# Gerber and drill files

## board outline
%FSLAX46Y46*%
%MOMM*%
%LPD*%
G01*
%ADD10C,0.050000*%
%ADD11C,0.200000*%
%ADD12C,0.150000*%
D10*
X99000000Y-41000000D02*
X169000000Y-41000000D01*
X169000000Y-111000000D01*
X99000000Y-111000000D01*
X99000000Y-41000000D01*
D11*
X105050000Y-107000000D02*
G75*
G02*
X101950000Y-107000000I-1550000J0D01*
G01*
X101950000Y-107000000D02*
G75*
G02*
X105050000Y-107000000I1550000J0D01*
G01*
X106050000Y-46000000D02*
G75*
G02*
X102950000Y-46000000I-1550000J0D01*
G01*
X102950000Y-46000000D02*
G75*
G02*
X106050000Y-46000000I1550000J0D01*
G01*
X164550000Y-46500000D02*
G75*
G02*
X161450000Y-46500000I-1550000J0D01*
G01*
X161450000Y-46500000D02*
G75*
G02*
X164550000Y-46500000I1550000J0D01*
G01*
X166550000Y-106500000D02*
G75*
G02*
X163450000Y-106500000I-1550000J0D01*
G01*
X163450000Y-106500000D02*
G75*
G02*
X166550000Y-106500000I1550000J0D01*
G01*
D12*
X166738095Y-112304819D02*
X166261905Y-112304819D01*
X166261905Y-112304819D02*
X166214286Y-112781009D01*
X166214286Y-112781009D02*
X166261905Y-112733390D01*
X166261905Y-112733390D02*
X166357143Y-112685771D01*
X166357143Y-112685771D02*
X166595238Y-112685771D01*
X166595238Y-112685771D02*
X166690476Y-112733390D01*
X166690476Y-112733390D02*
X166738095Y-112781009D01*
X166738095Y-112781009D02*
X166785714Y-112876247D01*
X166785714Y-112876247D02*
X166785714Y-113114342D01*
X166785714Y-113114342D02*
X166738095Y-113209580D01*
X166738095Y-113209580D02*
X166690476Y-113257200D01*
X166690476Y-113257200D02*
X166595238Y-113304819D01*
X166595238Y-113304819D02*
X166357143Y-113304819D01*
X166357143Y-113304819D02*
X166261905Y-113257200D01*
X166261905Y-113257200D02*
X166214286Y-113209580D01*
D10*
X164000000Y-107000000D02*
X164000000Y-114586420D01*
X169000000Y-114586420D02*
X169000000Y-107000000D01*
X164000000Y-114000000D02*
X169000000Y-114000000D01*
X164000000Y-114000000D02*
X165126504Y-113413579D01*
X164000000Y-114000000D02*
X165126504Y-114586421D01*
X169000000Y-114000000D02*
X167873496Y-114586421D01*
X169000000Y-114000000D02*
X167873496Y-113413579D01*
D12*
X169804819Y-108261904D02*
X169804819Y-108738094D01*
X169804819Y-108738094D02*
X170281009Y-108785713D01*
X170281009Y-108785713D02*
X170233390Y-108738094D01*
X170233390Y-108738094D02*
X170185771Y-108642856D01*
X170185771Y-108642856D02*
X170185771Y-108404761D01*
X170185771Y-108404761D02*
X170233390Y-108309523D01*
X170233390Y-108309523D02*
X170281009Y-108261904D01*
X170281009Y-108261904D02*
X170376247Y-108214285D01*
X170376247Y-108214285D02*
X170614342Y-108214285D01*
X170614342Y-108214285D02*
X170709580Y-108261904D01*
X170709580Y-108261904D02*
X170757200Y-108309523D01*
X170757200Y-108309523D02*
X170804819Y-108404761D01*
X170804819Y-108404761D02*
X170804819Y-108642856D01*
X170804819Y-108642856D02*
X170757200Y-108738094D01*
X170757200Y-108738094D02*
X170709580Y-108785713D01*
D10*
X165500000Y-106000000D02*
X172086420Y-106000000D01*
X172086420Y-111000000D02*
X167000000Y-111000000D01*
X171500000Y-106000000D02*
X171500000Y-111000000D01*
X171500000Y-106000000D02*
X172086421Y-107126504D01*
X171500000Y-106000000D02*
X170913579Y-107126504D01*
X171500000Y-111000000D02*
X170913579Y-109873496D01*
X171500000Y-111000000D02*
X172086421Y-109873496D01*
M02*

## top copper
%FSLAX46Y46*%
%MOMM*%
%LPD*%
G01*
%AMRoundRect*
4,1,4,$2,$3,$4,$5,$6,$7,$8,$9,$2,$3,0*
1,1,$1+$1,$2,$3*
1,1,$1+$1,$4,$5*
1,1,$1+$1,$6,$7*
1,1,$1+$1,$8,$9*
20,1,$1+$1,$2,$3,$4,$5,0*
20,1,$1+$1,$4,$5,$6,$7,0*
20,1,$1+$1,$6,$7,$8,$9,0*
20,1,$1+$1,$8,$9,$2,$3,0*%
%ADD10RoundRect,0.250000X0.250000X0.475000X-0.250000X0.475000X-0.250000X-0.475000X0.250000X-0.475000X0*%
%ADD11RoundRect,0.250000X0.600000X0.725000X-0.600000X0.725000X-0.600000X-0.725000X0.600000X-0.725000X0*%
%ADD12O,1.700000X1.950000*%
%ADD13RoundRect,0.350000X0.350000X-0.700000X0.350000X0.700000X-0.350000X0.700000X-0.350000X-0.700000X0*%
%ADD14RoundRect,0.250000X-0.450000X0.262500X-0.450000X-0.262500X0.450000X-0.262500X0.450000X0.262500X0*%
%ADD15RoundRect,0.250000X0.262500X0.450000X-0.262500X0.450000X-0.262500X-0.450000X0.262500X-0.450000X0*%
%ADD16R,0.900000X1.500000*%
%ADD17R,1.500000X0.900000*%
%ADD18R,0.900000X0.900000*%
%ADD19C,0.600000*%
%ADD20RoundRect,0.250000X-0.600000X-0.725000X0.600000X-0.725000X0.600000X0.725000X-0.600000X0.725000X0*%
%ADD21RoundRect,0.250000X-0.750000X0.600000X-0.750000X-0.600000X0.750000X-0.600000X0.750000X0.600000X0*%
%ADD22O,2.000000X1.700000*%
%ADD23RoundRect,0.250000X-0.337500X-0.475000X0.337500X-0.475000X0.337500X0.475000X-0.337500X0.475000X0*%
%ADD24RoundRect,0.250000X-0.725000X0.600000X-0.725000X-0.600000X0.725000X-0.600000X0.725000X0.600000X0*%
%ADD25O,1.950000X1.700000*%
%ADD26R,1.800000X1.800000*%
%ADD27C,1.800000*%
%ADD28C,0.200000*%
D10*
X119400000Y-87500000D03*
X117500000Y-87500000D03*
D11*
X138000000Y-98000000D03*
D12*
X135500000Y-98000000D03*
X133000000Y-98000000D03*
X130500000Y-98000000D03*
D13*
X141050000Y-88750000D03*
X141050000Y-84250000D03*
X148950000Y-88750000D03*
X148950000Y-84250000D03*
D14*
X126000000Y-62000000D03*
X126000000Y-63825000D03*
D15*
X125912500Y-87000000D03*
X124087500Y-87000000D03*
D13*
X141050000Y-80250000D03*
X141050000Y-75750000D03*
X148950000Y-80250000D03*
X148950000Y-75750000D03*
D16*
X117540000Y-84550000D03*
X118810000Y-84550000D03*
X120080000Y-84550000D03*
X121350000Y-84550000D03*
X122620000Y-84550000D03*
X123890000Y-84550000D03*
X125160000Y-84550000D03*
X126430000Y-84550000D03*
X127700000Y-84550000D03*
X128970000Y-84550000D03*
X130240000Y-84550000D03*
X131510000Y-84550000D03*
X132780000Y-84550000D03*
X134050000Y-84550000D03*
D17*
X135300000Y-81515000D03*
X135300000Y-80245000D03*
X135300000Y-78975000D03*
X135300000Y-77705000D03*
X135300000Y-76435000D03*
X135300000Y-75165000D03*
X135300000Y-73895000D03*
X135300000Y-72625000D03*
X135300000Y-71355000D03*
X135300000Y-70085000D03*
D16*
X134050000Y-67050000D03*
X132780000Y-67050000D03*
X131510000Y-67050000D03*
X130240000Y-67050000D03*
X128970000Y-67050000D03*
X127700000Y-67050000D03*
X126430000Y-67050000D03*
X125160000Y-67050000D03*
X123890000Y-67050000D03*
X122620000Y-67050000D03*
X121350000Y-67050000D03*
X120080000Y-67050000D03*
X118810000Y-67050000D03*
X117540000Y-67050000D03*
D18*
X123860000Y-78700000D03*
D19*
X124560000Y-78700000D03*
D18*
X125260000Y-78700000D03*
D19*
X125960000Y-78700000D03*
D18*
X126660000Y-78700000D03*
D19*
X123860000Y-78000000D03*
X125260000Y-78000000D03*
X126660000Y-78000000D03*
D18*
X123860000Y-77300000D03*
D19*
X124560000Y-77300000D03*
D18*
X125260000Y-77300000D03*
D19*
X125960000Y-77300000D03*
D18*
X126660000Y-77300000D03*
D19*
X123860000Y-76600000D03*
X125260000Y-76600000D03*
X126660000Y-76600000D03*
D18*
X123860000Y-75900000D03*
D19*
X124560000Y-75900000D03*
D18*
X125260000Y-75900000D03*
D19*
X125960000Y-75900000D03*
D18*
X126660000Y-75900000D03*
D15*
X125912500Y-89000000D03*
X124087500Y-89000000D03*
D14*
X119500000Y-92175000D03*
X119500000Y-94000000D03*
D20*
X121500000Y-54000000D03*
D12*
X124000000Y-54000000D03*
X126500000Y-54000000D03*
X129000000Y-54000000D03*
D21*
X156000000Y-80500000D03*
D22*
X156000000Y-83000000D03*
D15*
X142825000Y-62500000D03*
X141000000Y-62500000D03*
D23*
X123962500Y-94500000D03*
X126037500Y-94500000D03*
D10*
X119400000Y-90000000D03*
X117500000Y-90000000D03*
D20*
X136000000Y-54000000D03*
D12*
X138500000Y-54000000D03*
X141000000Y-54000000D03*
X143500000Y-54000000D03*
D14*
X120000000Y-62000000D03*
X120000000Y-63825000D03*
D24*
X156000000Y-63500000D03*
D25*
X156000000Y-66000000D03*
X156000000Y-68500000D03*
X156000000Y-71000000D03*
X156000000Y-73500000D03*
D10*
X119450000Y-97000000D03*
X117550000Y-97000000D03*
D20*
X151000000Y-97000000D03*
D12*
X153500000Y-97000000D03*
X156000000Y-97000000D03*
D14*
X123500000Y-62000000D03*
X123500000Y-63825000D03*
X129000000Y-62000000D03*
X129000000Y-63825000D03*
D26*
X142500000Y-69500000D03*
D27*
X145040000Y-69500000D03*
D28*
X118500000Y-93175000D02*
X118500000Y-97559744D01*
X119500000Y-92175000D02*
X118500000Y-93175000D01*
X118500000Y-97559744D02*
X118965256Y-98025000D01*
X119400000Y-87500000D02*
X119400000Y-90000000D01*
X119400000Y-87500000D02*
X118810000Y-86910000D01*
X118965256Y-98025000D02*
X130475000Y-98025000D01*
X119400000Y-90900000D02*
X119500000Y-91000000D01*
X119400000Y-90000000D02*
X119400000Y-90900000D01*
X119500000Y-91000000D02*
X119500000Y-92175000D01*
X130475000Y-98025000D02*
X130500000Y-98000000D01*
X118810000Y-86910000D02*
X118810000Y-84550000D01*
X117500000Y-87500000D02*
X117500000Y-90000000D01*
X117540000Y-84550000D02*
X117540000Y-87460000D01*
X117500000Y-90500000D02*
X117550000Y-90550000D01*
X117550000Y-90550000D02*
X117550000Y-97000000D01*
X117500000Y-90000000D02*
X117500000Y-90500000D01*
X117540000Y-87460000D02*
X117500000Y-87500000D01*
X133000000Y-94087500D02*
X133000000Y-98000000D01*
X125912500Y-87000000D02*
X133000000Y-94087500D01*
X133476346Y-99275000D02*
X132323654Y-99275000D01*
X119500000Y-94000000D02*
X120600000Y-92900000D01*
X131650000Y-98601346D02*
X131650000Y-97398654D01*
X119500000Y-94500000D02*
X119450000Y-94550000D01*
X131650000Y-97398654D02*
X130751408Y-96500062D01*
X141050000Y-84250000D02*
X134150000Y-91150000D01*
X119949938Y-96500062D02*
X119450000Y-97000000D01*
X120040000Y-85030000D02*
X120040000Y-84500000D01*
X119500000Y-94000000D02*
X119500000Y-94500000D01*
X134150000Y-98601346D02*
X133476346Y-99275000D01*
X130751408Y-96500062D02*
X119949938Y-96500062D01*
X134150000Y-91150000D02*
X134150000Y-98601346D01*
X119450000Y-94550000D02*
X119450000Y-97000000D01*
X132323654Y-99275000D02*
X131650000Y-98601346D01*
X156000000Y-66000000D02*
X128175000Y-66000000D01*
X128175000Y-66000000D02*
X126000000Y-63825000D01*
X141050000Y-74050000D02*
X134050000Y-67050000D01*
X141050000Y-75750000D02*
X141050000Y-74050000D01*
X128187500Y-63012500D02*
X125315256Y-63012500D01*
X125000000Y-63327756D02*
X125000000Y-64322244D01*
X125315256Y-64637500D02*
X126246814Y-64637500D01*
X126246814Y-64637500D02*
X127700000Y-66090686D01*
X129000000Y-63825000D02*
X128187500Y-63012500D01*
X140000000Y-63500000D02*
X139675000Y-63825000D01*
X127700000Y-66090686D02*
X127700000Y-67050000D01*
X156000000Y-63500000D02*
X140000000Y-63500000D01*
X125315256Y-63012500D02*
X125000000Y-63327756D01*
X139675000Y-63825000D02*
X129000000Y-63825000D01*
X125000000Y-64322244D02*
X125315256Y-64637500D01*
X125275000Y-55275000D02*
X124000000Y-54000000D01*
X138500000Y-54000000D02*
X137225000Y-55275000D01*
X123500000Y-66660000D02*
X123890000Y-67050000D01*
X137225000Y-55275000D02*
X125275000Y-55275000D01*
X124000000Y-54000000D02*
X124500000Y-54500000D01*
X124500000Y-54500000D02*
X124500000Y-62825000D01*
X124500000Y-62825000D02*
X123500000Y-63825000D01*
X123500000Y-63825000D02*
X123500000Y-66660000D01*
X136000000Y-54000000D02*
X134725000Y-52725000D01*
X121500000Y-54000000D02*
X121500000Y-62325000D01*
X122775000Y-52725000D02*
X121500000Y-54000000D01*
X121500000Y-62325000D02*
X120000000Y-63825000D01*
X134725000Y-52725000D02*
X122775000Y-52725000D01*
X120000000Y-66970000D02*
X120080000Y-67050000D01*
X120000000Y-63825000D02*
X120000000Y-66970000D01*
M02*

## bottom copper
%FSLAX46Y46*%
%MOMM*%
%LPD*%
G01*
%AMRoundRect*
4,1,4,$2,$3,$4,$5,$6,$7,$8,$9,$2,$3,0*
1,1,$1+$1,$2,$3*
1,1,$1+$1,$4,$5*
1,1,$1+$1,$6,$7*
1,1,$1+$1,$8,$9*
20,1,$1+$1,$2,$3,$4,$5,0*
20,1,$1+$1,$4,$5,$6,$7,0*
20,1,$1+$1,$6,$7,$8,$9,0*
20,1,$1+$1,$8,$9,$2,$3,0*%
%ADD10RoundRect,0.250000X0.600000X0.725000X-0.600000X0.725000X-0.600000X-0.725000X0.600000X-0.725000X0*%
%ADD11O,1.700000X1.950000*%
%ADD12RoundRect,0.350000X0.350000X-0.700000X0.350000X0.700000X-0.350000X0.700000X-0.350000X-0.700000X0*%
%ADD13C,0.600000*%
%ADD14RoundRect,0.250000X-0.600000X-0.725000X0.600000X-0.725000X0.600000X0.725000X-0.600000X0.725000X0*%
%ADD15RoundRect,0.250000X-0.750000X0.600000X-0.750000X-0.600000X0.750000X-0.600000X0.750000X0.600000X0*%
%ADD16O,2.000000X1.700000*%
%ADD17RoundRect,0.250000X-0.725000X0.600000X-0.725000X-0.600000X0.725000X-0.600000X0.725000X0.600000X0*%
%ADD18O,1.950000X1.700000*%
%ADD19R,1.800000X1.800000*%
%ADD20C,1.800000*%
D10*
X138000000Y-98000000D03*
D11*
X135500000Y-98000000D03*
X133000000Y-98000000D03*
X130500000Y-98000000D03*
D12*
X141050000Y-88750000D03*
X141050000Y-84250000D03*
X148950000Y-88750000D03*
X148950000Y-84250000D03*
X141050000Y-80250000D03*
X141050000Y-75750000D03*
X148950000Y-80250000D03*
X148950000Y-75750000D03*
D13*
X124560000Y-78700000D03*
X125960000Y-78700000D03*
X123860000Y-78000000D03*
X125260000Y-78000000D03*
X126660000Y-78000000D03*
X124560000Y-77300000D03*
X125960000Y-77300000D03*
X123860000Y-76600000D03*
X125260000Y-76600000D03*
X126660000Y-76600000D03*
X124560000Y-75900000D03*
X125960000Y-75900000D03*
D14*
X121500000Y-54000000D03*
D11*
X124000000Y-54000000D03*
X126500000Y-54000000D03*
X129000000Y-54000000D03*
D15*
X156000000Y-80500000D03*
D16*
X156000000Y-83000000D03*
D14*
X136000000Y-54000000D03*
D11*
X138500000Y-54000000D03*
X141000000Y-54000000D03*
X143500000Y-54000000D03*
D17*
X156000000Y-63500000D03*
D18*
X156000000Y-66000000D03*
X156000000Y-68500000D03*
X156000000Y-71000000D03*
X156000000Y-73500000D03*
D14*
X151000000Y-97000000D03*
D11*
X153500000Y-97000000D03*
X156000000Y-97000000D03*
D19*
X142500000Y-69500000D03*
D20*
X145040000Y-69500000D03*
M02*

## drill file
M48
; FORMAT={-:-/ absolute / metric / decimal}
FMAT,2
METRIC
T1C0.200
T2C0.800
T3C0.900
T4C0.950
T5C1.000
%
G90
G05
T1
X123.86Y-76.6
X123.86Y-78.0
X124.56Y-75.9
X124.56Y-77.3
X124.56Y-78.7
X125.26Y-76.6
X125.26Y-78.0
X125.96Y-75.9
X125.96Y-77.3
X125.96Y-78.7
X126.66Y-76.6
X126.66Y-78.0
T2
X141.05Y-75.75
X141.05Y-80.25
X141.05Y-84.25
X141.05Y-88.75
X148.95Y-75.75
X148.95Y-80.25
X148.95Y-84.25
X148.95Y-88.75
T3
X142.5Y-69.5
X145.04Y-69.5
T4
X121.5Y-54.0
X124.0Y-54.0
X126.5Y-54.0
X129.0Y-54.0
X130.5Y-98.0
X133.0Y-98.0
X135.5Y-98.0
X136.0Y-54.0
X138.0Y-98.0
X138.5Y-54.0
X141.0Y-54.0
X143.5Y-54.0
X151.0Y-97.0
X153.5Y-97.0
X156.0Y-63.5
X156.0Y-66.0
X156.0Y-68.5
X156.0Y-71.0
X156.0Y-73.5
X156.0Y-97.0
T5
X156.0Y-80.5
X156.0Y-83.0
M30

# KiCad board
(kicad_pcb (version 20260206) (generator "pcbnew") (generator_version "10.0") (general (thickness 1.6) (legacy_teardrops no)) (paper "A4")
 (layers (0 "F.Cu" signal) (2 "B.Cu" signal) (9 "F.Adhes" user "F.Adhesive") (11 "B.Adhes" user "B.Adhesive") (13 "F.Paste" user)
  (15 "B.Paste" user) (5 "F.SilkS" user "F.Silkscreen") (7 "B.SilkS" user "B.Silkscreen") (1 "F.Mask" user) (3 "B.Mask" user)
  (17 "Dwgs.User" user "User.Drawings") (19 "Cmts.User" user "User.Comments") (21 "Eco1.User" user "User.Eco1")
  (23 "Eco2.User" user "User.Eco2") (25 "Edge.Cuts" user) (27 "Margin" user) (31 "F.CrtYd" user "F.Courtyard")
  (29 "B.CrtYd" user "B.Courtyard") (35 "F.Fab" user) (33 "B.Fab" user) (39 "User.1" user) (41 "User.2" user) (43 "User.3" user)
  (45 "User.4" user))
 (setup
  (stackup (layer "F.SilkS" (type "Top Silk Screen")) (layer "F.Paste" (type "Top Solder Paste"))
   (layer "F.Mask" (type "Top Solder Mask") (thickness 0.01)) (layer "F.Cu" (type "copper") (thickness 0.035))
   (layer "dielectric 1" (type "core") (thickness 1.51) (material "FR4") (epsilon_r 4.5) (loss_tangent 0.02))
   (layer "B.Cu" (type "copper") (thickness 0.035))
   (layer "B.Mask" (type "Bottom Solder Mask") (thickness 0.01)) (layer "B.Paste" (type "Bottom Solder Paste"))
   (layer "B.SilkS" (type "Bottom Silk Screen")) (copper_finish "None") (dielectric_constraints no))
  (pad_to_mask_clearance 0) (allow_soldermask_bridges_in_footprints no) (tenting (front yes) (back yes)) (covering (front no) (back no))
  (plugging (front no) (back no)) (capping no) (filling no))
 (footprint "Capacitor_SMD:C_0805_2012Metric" (layer "F.Cu") (at 118.45 87.5 180)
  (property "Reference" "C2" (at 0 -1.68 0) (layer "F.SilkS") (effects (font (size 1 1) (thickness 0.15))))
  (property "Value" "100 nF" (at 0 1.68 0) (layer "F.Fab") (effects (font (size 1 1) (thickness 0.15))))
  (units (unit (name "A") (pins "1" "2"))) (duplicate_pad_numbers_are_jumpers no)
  (pad "1" smd roundrect (at -0.95 0 180) (size 1 1.45) (layers "F.Cu" "F.Mask" "F.Paste") (roundrect_rratio 0.25) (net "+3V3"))
  (pad "2" smd roundrect (at 0.95 0 180) (size 1 1.45) (layers "F.Cu" "F.Mask" "F.Paste") (roundrect_rratio 0.25) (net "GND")))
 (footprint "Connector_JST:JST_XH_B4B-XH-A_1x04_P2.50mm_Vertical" (layer "F.Cu") (at 138 98 180)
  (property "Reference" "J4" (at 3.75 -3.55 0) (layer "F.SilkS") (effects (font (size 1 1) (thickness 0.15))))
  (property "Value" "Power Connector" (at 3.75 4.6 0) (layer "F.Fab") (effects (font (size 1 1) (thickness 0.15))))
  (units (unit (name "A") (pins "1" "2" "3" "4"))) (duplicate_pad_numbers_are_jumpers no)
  (pad "1" thru_hole roundrect (at 0 0 180) (size 1.7 1.95) (drill 0.95) (layers "*.Cu" "*.Mask") (remove_unused_layers no)
   (roundrect_rratio 0.147059) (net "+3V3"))
  (pad "2" thru_hole oval (at 2.5 0 180) (size 1.7 1.95) (drill 0.95) (layers "*.Cu" "*.Mask") (remove_unused_layers no) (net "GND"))
  (pad "3" thru_hole oval (at 5 0 180) (size 1.7 1.95) (drill 0.95) (layers "*.Cu" "*.Mask") (remove_unused_layers no) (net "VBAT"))
  (pad "4" thru_hole oval (at 7.5 0 180) (size 1.7 1.95) (drill 0.95) (layers "*.Cu" "*.Mask") (remove_unused_layers no) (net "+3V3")))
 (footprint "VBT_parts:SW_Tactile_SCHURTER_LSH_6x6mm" (layer "F.Cu") (at 145 86.5)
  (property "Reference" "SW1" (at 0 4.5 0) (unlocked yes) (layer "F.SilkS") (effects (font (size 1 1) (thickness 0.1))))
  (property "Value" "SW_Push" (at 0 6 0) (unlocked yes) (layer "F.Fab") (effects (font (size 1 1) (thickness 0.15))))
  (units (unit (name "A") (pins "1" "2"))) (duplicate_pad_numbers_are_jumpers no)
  (pad "1" thru_hole roundrect (at -3.95 2.25 90) (size 2.1 1.4) (drill 0.8) (layers "*.Cu" "*.Mask") (remove_unused_layers no)
   (roundrect_rratio 0.25) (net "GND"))
  (pad "2" thru_hole roundrect (at -3.95 -2.25 90) (size 2.1 1.4) (drill 0.8) (layers "*.Cu" "*.Mask") (remove_unused_layers no)
   (roundrect_rratio 0.25) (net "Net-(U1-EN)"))
  (pad "3" thru_hole roundrect (at 3.95 2.25 90) (size 2.1 1.4) (drill 0.8) (layers "*.Cu" "*.Mask") (remove_unused_layers no)
   (roundrect_rratio 0.25))
  (pad "4" thru_hole roundrect (at 3.95 -2.25 90) (size 2.1 1.4) (drill 0.8) (layers "*.Cu" "*.Mask") (remove_unused_layers no)
   (roundrect_rratio 0.25)))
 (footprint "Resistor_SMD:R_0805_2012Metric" (layer "F.Cu") (at 126 62.9125 -90)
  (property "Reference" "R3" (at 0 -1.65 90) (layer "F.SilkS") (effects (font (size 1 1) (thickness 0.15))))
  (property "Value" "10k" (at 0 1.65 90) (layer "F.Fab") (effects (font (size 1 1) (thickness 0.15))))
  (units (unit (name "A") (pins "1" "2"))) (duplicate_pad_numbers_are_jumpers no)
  (pad "1" smd roundrect (at -0.9125 0 270) (size 1.025 1.4) (layers "F.Cu" "F.Mask" "F.Paste") (roundrect_rratio 0.243902) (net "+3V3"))
  (pad "2" smd roundrect (at 0.9125 0 270) (size 1.025 1.4) (layers "F.Cu" "F.Mask" "F.Paste") (roundrect_rratio 0.243902) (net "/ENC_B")))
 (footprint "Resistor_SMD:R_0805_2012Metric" (layer "F.Cu") (at 125 87 180)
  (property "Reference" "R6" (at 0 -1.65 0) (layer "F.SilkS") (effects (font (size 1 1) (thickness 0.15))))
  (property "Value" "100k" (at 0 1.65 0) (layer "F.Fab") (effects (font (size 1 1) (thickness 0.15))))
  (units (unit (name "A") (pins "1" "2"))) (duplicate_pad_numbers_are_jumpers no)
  (pad "1" smd roundrect (at -0.9125 0 180) (size 1.025 1.4) (layers "F.Cu" "F.Mask" "F.Paste") (roundrect_rratio 0.243902) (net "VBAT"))
  (pad "2" smd roundrect (at 0.9125 0 180) (size 1.025 1.4) (layers "F.Cu" "F.Mask" "F.Paste") (roundrect_rratio 0.243902)
   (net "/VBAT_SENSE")))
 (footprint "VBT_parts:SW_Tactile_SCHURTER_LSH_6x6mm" (layer "F.Cu") (at 145 78)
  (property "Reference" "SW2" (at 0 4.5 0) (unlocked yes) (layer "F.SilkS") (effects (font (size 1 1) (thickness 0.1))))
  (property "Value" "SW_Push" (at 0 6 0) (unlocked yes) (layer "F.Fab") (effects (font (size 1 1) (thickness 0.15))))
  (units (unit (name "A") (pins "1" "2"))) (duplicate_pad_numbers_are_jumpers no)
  (pad "1" thru_hole roundrect (at -3.95 2.25 90) (size 2.1 1.4) (drill 0.8) (layers "*.Cu" "*.Mask") (remove_unused_layers no)
   (roundrect_rratio 0.25) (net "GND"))
  (pad "2" thru_hole roundrect (at -3.95 -2.25 90) (size 2.1 1.4) (drill 0.8) (layers "*.Cu" "*.Mask") (remove_unused_layers no)
   (roundrect_rratio 0.25) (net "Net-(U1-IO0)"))
  (pad "3" thru_hole roundrect (at 3.95 2.25 90) (size 2.1 1.4) (drill 0.8) (layers "*.Cu" "*.Mask") (remove_unused_layers no)
   (roundrect_rratio 0.25))
  (pad "4" thru_hole roundrect (at 3.95 -2.25 90) (size 2.1 1.4) (drill 0.8) (layers "*.Cu" "*.Mask") (remove_unused_layers no)
   (roundrect_rratio 0.25)))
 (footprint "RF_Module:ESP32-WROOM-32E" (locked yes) (layer "F.Cu") (at 122.8 75.8 90)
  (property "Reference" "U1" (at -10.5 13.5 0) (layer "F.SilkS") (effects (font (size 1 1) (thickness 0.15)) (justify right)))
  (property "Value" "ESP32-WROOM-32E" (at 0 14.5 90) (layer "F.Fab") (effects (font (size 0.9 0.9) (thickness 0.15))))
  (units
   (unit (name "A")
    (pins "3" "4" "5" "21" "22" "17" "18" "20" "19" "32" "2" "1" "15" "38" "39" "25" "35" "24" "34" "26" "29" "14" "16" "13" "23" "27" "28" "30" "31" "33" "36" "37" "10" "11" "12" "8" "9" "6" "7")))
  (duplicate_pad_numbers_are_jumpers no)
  (pad "1" smd rect (at -8.75 -5.26 90) (size 1.5 0.9) (layers "F.Cu" "F.Mask" "F.Paste") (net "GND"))
  (pad "2" smd rect (at -8.75 -3.99 90) (size 1.5 0.9) (layers "F.Cu" "F.Mask" "F.Paste") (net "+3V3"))
  (pad "3" smd rect (at -8.75 -2.72 90) (size 1.5 0.9) (layers "F.Cu" "F.Mask" "F.Paste") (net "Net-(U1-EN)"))
  (pad "4" smd rect (at -8.75 -1.45 90) (size 1.5 0.9) (layers "F.Cu" "F.Mask" "F.Paste") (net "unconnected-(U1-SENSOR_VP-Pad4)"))
  (pad "5" smd rect (at -8.75 -0.18 90) (size 1.5 0.9) (layers "F.Cu" "F.Mask" "F.Paste") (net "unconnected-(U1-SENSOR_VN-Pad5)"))
  (pad "6" smd rect (at -8.75 1.09 90) (size 1.5 0.9) (layers "F.Cu" "F.Mask" "F.Paste") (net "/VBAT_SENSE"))
  (pad "7" smd rect (at -8.75 2.36 90) (size 1.5 0.9) (layers "F.Cu" "F.Mask" "F.Paste") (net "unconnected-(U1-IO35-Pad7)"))
  (pad "8" smd rect (at -8.75 3.63 90) (size 1.5 0.9) (layers "F.Cu" "F.Mask" "F.Paste") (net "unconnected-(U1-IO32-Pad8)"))
  (pad "9" smd rect (at -8.75 4.9 90) (size 1.5 0.9) (layers "F.Cu" "F.Mask" "F.Paste") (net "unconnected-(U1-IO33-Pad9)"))
  (pad "10" smd rect (at -8.75 6.17 90) (size 1.5 0.9) (layers "F.Cu" "F.Mask" "F.Paste") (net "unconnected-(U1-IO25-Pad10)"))
  (pad "11" smd rect (at -8.75 7.44 90) (size 1.5 0.9) (layers "F.Cu" "F.Mask" "F.Paste") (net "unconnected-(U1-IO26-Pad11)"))
  (pad "12" smd rect (at -8.75 8.71 90) (size 1.5 0.9) (layers "F.Cu" "F.Mask" "F.Paste") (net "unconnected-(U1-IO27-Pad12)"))
  (pad "13" smd rect (at -8.75 9.98 90) (size 1.5 0.9) (layers "F.Cu" "F.Mask" "F.Paste") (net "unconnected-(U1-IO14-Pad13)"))
  (pad "14" smd rect (at -8.75 11.25 90) (size 1.5 0.9) (layers "F.Cu" "F.Mask" "F.Paste") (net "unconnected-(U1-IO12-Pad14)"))
  (pad "15" smd rect (at -5.715 12.5 180) (size 1.5 0.9) (layers "F.Cu" "F.Mask" "F.Paste") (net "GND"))
  (pad "16" smd rect (at -4.445 12.5 180) (size 1.5 0.9) (layers "F.Cu" "F.Mask" "F.Paste") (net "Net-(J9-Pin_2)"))
  (pad "17" smd rect (at -3.175 12.5 180) (size 1.5 0.9) (layers "F.Cu" "F.Mask" "F.Paste") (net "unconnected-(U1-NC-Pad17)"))
  (pad "18" smd rect (at -1.905 12.5 180) (size 1.5 0.9) (layers "F.Cu" "F.Mask" "F.Paste") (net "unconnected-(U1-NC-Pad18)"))
  (pad "19" smd rect (at -0.635 12.5 180) (size 1.5 0.9) (layers "F.Cu" "F.Mask" "F.Paste") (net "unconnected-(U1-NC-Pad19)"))
  (pad "20" smd rect (at 0.635 12.5 180) (size 1.5 0.9) (layers "F.Cu" "F.Mask" "F.Paste") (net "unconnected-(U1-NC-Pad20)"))
  (pad "21" smd rect (at 1.905 12.5 180) (size 1.5 0.9) (layers "F.Cu" "F.Mask" "F.Paste") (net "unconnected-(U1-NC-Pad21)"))
  (pad "22" smd rect (at 3.175 12.5 180) (size 1.5 0.9) (layers "F.Cu" "F.Mask" "F.Paste") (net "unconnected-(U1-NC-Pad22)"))
  (pad "23" smd rect (at 4.445 12.5 180) (size 1.5 0.9) (layers "F.Cu" "F.Mask" "F.Paste") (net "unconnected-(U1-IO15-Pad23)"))
  (pad "24" smd rect (at 5.715 12.5 180) (size 1.5 0.9) (layers "F.Cu" "F.Mask" "F.Paste") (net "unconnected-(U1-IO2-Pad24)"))
  (pad "25" smd rect (at 8.75 11.25 90) (size 1.5 0.9) (layers "F.Cu" "F.Mask" "F.Paste") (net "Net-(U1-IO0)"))
  (pad "26" smd rect (at 8.75 9.98 90) (size 1.5 0.9) (layers "F.Cu" "F.Mask" "F.Paste") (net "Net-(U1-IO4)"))
  (pad "27" smd rect (at 8.75 8.71 90) (size 1.5 0.9) (layers "F.Cu" "F.Mask" "F.Paste") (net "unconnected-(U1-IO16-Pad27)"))
  (pad "28" smd rect (at 8.75 7.44 90) (size 1.5 0.9) (layers "F.Cu" "F.Mask" "F.Paste") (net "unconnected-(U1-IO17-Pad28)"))
  (pad "29" smd rect (at 8.75 6.17 90) (size 1.5 0.9) (layers "F.Cu" "F.Mask" "F.Paste") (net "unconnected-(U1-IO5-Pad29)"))
  (pad "30" smd rect (at 8.75 4.9 90) (size 1.5 0.9) (layers "F.Cu" "F.Mask" "F.Paste") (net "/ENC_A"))
  (pad "31" smd rect (at 8.75 3.63 90) (size 1.5 0.9) (layers "F.Cu" "F.Mask" "F.Paste") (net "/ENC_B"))
  (pad "32" smd rect (at 8.75 2.36 90) (size 1.5 0.9) (layers "F.Cu" "F.Mask" "F.Paste") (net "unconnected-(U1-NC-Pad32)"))
  (pad "33" smd rect (at 8.75 1.09 90) (size 1.5 0.9) (layers "F.Cu" "F.Mask" "F.Paste") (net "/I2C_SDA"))
  (pad "34" smd rect (at 8.75 -0.18 90) (size 1.5 0.9) (layers "F.Cu" "F.Mask" "F.Paste") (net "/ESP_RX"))
  (pad "35" smd rect (at 8.75 -1.45 90) (size 1.5 0.9) (layers "F.Cu" "F.Mask" "F.Paste") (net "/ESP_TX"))
  (pad "36" smd rect (at 8.75 -2.72 90) (size 1.5 0.9) (layers "F.Cu" "F.Mask" "F.Paste") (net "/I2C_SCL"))
  (pad "37" smd rect (at 8.75 -3.99 90) (size 1.5 0.9) (layers "F.Cu" "F.Mask" "F.Paste") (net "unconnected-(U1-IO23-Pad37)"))
  (pad "38" smd rect (at 8.75 -5.26 90) (size 1.5 0.9) (layers "F.Cu" "F.Mask" "F.Paste") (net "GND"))
  (pad "39" smd rect (at -2.9 1.06 90) (size 0.9 0.9) (layers "F.Cu" "F.Mask" "F.Paste") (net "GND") (zone_connect 2))
  (pad "39" thru_hole circle (at -2.9 1.76 90) (size 0.6 0.6) (drill 0.2) (layers "*.Cu" "*.Mask") (remove_unused_layers no) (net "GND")
   (zone_connect 2))
  (pad "39" smd rect (at -2.9 2.46 90) (size 0.9 0.9) (layers "F.Cu" "F.Mask" "F.Paste") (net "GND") (zone_connect 2))
  (pad "39" thru_hole circle (at -2.9 3.16 90) (size 0.6 0.6) (drill 0.2) (layers "*.Cu" "*.Mask") (remove_unused_layers no) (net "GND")
   (zone_connect 2))
  (pad "39" smd rect (at -2.9 3.86 90) (size 0.9 0.9) (layers "F.Cu" "F.Mask" "F.Paste") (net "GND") (zone_connect 2))
  (pad "39" thru_hole circle (at -2.2 1.06 90) (size 0.6 0.6) (drill 0.2) (layers "*.Cu" "*.Mask") (remove_unused_layers no) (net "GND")
   (zone_connect 2))
  (pad "39" thru_hole circle (at -2.2 2.46 90) (size 0.6 0.6) (drill 0.2) (layers "*.Cu" "*.Mask") (remove_unused_layers no) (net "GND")
   (zone_connect 2))
  (pad "39" thru_hole circle (at -2.2 3.86 90) (size 0.6 0.6) (drill 0.2) (layers "*.Cu" "*.Mask") (remove_unused_layers no) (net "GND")
   (zone_connect 2))
  (pad "39" smd rect (at -1.5 1.06 90) (size 0.9 0.9) (layers "F.Cu" "F.Mask" "F.Paste") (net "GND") (zone_connect 2))
  (pad "39" thru_hole circle (at -1.5 1.76 90) (size 0.6 0.6) (drill 0.2) (layers "*.Cu" "*.Mask") (remove_unused_layers no) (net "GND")
   (zone_connect 2))
  (pad "39" smd rect (at -1.5 2.46 90) (size 0.9 0.9) (layers "F.Cu" "F.Mask" "F.Paste") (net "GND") (zone_connect 2))
  (pad "39" thru_hole circle (at -1.5 3.16 90) (size 0.6 0.6) (drill 0.2) (layers "*.Cu" "*.Mask") (remove_unused_layers no) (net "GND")
   (zone_connect 2))
  (pad "39" smd rect (at -1.5 3.86 90) (size 0.9 0.9) (layers "F.Cu" "F.Mask" "F.Paste") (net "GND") (zone_connect 2))
  (pad "39" thru_hole circle (at -0.8 1.06 90) (size 0.6 0.6) (drill 0.2) (layers "*.Cu" "*.Mask") (remove_unused_layers no) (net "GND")
   (zone_connect 2))
  (pad "39" thru_hole circle (at -0.8 2.46 90) (size 0.6 0.6) (drill 0.2) (layers "*.Cu" "*.Mask") (remove_unused_layers no) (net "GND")
   (zone_connect 2))
  (pad "39" thru_hole circle (at -0.8 3.86 90) (size 0.6 0.6) (drill 0.2) (layers "*.Cu" "*.Mask") (remove_unused_layers no) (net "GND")
   (zone_connect 2))
  (pad "39" smd rect (at -0.1 1.06 90) (size 0.9 0.9) (layers "F.Cu" "F.Mask" "F.Paste") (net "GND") (zone_connect 2))
  (pad "39" thru_hole circle (at -0.1 1.76 90) (size 0.6 0.6) (drill 0.2) (layers "*.Cu" "*.Mask") (remove_unused_layers no) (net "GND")
   (zone_connect 2))
  (pad "39" smd rect (at -0.1 2.46 90) (size 0.9 0.9) (layers "F.Cu" "F.Mask" "F.Paste") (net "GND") (zone_connect 2))
  (pad "39" thru_hole circle (at -0.1 3.16 90) (size 0.6 0.6) (drill 0.2) (layers "*.Cu" "*.Mask") (remove_unused_layers no) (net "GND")
   (zone_connect 2))
  (pad "39" smd rect (at -0.1 3.86 90) (size 0.9 0.9) (layers "F.Cu" "F.Mask" "F.Paste") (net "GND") (zone_connect 2))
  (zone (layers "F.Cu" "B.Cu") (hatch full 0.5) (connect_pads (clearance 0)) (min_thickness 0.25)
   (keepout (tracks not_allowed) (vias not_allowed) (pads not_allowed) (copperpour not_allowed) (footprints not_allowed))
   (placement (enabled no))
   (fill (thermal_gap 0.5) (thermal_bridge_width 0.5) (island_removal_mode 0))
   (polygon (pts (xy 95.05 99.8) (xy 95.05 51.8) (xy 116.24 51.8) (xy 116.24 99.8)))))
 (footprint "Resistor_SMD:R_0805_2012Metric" (layer "F.Cu") (at 125 89 180)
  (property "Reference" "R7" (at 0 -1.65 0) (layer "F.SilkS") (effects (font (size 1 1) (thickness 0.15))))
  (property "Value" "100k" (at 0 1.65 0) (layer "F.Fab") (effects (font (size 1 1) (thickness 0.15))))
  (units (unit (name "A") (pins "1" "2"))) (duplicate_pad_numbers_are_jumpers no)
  (pad "1" smd roundrect (at -0.9125 0 180) (size 1.025 1.4) (layers "F.Cu" "F.Mask" "F.Paste") (roundrect_rratio 0.243902) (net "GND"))
  (pad "2" smd roundrect (at 0.9125 0 180) (size 1.025 1.4) (layers "F.Cu" "F.Mask" "F.Paste") (roundrect_rratio 0.243902)
   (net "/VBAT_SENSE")))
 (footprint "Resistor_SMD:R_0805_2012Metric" (layer "F.Cu") (at 119.5 93.0875 -90)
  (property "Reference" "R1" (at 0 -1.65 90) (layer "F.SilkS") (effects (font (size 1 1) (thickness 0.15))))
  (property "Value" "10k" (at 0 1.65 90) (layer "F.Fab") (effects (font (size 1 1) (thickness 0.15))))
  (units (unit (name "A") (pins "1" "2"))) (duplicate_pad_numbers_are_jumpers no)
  (pad "1" smd roundrect (at -0.9125 0 270) (size 1.025 1.4) (layers "F.Cu" "F.Mask" "F.Paste") (roundrect_rratio 0.243902) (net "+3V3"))
  (pad "2" smd roundrect (at 0.9125 0 270) (size 1.025 1.4) (layers "F.Cu" "F.Mask" "F.Paste") (roundrect_rratio 0.243902)
   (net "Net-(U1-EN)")))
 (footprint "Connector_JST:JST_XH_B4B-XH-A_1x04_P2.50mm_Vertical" (layer "F.Cu") (at 121.5 54)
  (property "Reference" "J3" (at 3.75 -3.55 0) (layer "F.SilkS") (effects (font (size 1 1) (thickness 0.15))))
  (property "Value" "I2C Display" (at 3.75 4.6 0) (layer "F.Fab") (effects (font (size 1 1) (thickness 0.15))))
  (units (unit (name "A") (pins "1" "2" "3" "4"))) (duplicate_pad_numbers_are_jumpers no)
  (pad "1" thru_hole roundrect (at 0 0) (size 1.7 1.95) (drill 0.95) (layers "*.Cu" "*.Mask") (remove_unused_layers no)
   (roundrect_rratio 0.147059) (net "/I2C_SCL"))
  (pad "2" thru_hole oval (at 2.5 0) (size 1.7 1.95) (drill 0.95) (layers "*.Cu" "*.Mask") (remove_unused_layers no) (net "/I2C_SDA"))
  (pad "3" thru_hole oval (at 5 0) (size 1.7 1.95) (drill 0.95) (layers "*.Cu" "*.Mask") (remove_unused_layers no) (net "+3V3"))
  (pad "4" thru_hole oval (at 7.5 0) (size 1.7 1.95) (drill 0.95) (layers "*.Cu" "*.Mask") (remove_unused_layers no) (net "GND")))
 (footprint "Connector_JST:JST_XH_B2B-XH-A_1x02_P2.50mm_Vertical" (layer "F.Cu") (at 156 80.5 -90)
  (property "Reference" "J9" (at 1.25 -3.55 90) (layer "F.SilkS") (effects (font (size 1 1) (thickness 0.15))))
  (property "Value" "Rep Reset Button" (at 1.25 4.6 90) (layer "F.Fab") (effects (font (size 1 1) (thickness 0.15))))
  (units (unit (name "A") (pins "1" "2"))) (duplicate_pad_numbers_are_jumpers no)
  (pad "1" thru_hole roundrect (at 0 0 270) (size 1.7 2) (drill 1) (layers "*.Cu" "*.Mask") (remove_unused_layers no)
   (roundrect_rratio 0.147059) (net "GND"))
  (pad "2" thru_hole oval (at 2.5 0 270) (size 1.7 2) (drill 1) (layers "*.Cu" "*.Mask") (remove_unused_layers no) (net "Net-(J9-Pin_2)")))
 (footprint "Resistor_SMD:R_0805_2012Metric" (layer "F.Cu") (at 141.9125 62.5 180)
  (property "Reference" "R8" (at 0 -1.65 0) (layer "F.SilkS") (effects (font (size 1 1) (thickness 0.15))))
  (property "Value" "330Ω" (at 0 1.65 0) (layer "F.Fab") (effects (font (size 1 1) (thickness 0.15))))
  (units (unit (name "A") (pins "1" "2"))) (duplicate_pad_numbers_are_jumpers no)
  (pad "1" smd roundrect (at -0.9125 0 180) (size 1.025 1.4) (layers "F.Cu" "F.Mask" "F.Paste") (roundrect_rratio 0.243902)
   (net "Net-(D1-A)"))
  (pad "2" smd roundrect (at 0.9125 0 180) (size 1.025 1.4) (layers "F.Cu" "F.Mask" "F.Paste") (roundrect_rratio 0.243902)
   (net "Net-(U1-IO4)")))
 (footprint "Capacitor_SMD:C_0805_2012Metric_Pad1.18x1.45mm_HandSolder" (layer "F.Cu") (at 125 94.5)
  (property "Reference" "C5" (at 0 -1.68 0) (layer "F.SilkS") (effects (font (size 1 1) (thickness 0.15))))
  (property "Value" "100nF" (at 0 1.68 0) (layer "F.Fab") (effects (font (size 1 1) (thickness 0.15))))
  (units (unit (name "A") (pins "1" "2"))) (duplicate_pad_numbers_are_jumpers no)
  (pad "1" smd roundrect (at -1.0375 0) (size 1.175 1.45) (layers "F.Cu" "F.Mask" "F.Paste") (roundrect_rratio 0.212766) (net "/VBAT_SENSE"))
  (pad "2" smd roundrect (at 1.0375 0) (size 1.175 1.45) (layers "F.Cu" "F.Mask" "F.Paste") (roundrect_rratio 0.212766) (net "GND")))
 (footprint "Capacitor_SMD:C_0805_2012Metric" (layer "F.Cu") (at 118.45 90 180)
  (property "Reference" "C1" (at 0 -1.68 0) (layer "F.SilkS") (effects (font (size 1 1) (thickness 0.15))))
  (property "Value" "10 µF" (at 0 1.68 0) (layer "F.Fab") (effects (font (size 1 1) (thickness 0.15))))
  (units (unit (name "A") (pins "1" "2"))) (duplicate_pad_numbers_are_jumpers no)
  (pad "1" smd roundrect (at -0.95 0 180) (size 1 1.45) (layers "F.Cu" "F.Mask" "F.Paste") (roundrect_rratio 0.25) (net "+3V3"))
  (pad "2" smd roundrect (at 0.95 0 180) (size 1 1.45) (layers "F.Cu" "F.Mask" "F.Paste") (roundrect_rratio 0.25) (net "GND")))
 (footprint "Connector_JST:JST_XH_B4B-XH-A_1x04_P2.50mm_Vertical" (layer "F.Cu") (at 136 54)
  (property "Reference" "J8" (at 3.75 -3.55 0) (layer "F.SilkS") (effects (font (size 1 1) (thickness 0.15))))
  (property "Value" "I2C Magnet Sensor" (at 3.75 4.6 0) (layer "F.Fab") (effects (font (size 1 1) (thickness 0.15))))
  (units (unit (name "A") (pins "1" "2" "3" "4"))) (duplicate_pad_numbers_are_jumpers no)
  (pad "1" thru_hole roundrect (at 0 0) (size 1.7 1.95) (drill 0.95) (layers "*.Cu" "*.Mask") (remove_unused_layers no)
   (roundrect_rratio 0.147059) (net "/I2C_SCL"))
  (pad "2" thru_hole oval (at 2.5 0) (size 1.7 1.95) (drill 0.95) (layers "*.Cu" "*.Mask") (remove_unused_layers no) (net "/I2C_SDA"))
  (pad "3" thru_hole oval (at 5 0) (size 1.7 1.95) (drill 0.95) (layers "*.Cu" "*.Mask") (remove_unused_layers no) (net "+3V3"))
  (pad "4" thru_hole oval (at 7.5 0) (size 1.7 1.95) (drill 0.95) (layers "*.Cu" "*.Mask") (remove_unused_layers no) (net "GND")))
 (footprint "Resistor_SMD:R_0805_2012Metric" (layer "F.Cu") (at 120 62.9125 -90)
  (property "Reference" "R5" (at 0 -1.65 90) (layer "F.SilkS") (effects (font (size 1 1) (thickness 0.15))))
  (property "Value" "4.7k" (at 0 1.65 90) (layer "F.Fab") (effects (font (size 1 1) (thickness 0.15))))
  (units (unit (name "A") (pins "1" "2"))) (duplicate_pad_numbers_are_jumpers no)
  (pad "1" smd roundrect (at -0.9125 0 270) (size 1.025 1.4) (layers "F.Cu" "F.Mask" "F.Paste") (roundrect_rratio 0.243902) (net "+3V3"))
  (pad "2" smd roundrect (at 0.9125 0 270) (size 1.025 1.4) (layers "F.Cu" "F.Mask" "F.Paste") (roundrect_rratio 0.243902) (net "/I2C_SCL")))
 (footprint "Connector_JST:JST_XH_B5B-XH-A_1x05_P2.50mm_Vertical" (layer "F.Cu") (at 156 63.5 -90)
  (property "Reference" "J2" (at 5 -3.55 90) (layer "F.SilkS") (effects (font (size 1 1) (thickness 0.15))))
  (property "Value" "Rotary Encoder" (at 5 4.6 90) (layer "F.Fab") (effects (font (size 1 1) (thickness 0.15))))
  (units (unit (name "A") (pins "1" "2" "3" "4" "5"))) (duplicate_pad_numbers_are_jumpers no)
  (pad "1" thru_hole roundrect (at 0 0 270) (size 1.7 1.95) (drill 0.95) (layers "*.Cu" "*.Mask") (remove_unused_layers no)
   (roundrect_rratio 0.147059) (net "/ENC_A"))
  (pad "2" thru_hole oval (at 2.5 0 270) (size 1.7 1.95) (drill 0.95) (layers "*.Cu" "*.Mask") (remove_unused_layers no) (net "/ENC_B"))
  (pad "3" thru_hole oval (at 5 0 270) (size 1.7 1.95) (drill 0.95) (layers "*.Cu" "*.Mask") (remove_unused_layers no) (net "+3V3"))
  (pad "4" thru_hole oval (at 7.5 0 270) (size 1.7 1.95) (drill 0.95) (layers "*.Cu" "*.Mask") (remove_unused_layers no) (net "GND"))
  (pad "5" thru_hole oval (at 10 0 270) (size 1.7 1.95) (drill 0.95) (layers "*.Cu" "*.Mask") (remove_unused_layers no) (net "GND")))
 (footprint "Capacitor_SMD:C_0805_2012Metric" (layer "F.Cu") (at 118.5 97 180)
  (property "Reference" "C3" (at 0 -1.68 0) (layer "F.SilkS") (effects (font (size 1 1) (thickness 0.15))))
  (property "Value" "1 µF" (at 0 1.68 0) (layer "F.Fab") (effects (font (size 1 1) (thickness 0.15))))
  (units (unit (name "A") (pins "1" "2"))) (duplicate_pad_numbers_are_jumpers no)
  (pad "1" smd roundrect (at -0.95 0 180) (size 1 1.45) (layers "F.Cu" "F.Mask" "F.Paste") (roundrect_rratio 0.25) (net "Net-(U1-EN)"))
  (pad "2" smd roundrect (at 0.95 0 180) (size 1 1.45) (layers "F.Cu" "F.Mask" "F.Paste") (roundrect_rratio 0.25) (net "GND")))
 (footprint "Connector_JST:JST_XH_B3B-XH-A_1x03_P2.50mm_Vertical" (layer "F.Cu") (at 151 97)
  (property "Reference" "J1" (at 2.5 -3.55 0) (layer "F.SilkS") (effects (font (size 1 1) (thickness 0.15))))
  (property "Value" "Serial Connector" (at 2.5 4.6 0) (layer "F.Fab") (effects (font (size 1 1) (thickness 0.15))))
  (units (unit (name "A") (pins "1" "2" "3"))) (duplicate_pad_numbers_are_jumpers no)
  (pad "1" thru_hole roundrect (at 0 0) (size 1.7 1.95) (drill 0.95) (layers "*.Cu" "*.Mask") (remove_unused_layers no)
   (roundrect_rratio 0.147059) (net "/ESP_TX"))
  (pad "2" thru_hole oval (at 2.5 0) (size 1.7 1.95) (drill 0.95) (layers "*.Cu" "*.Mask") (remove_unused_layers no) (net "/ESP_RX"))
  (pad "3" thru_hole oval (at 5 0) (size 1.7 1.95) (drill 0.95) (layers "*.Cu" "*.Mask") (remove_unused_layers no) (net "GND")))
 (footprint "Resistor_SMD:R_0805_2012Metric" (layer "F.Cu") (at 123.5 62.9125 -90)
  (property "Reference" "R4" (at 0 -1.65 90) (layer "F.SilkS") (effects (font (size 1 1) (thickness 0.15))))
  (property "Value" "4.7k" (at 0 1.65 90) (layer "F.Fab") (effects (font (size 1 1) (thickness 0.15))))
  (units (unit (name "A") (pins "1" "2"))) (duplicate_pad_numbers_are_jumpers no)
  (pad "1" smd roundrect (at -0.9125 0 270) (size 1.025 1.4) (layers "F.Cu" "F.Mask" "F.Paste") (roundrect_rratio 0.243902) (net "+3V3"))
  (pad "2" smd roundrect (at 0.9125 0 270) (size 1.025 1.4) (layers "F.Cu" "F.Mask" "F.Paste") (roundrect_rratio 0.243902) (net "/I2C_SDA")))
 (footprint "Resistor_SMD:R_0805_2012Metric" (layer "F.Cu") (at 129 62.9125 -90)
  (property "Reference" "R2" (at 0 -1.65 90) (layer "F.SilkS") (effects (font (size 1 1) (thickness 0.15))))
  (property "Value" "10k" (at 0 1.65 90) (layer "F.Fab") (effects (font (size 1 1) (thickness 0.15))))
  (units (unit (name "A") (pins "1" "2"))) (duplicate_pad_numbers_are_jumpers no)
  (pad "1" smd roundrect (at -0.9125 0 270) (size 1.025 1.4) (layers "F.Cu" "F.Mask" "F.Paste") (roundrect_rratio 0.243902) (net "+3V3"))
  (pad "2" smd roundrect (at 0.9125 0 270) (size 1.025 1.4) (layers "F.Cu" "F.Mask" "F.Paste") (roundrect_rratio 0.243902) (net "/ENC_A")))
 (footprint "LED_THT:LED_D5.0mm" (layer "F.Cu") (at 142.5 69.5)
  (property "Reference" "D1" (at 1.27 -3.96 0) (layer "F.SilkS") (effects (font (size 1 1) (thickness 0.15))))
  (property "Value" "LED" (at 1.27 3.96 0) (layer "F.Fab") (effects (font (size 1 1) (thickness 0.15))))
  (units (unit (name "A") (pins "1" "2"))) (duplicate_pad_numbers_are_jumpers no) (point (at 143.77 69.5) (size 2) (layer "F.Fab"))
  (pad "1" thru_hole rect (at 0 0) (size 1.8 1.8) (drill 0.9) (layers "*.Cu" "*.Mask") (remove_unused_layers no) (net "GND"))
  (pad "2" thru_hole circle (at 2.54 0) (size 1.8 1.8) (drill 0.9) (layers "*.Cu" "*.Mask") (remove_unused_layers no) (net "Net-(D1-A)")))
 (gr_rect (start 99 41) (end 169 111) (stroke (width 0.05) (type default)) (fill no) (layer "Edge.Cuts"))
 (gr_circle (center 103.5 107) (end 105.05 107) (stroke (width 0.2) (type solid)) (fill no) (layer "Edge.Cuts"))
 (gr_circle (center 104.5 46) (end 106.05 46) (stroke (width 0.2) (type solid)) (fill no) (layer "Edge.Cuts"))
 (gr_circle (center 163 46.5) (end 164.55 46.5) (stroke (width 0.2) (type solid)) (fill no) (layer "Edge.Cuts"))
 (gr_circle (center 165 106.5) (end 166.55 106.5) (stroke (width 0.2) (type solid)) (fill no) (layer "Edge.Cuts"))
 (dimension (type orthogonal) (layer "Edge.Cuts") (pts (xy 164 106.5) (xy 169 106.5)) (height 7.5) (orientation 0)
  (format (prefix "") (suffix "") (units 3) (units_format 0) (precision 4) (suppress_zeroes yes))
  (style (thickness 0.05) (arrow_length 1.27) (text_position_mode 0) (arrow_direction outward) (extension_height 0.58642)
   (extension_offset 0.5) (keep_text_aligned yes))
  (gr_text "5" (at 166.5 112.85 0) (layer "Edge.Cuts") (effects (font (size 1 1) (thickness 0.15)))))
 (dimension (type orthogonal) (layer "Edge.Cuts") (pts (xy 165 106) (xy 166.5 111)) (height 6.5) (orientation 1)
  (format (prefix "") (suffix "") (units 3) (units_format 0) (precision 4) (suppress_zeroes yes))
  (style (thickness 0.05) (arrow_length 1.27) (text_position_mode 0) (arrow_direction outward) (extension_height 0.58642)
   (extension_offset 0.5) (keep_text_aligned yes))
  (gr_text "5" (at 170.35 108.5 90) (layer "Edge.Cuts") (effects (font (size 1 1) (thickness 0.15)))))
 (segment (start 118.5 93.175) (end 118.5 97.559744) (width 0.2) (layer "F.Cu") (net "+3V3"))
 (segment (start 119.5 92.175) (end 118.5 93.175) (width 0.2) (layer "F.Cu") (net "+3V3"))
 (segment (start 118.5 97.559744) (end 118.965256 98.025) (width 0.2) (layer "F.Cu") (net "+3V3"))
 (segment (start 119.4 87.5) (end 119.4 90) (width 0.2) (layer "F.Cu") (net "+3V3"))
 (segment (start 119.4 87.5) (end 118.81 86.91) (width 0.2) (layer "F.Cu") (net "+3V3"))
 (segment (start 118.965256 98.025) (end 130.475 98.025) (width 0.2) (layer "F.Cu") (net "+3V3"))
 (segment (start 119.4 90.9) (end 119.5 91) (width 0.2) (layer "F.Cu") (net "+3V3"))
 (segment (start 119.4 90) (end 119.4 90.9) (width 0.2) (layer "F.Cu") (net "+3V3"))
 (segment (start 119.5 91) (end 119.5 92.175) (width 0.2) (layer "F.Cu") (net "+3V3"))
 (segment (start 130.475 98.025) (end 130.5 98) (width 0.2) (layer "F.Cu") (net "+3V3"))
 (segment (start 118.81 86.91) (end 118.81 84.55) (width 0.2) (layer "F.Cu") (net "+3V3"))
 (segment (start 117.5 87.5) (end 117.5 90) (width 0.2) (layer "F.Cu") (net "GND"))
 (segment (start 117.54 84.55) (end 117.54 87.46) (width 0.2) (layer "F.Cu") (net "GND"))
 (segment (start 117.5 90.5) (end 117.55 90.55) (width 0.2) (layer "F.Cu") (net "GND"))
 (segment (start 117.55 90.55) (end 117.55 97) (width 0.2) (layer "F.Cu") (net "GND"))
 (segment (start 117.5 90) (end 117.5 90.5) (width 0.2) (layer "F.Cu") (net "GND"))
 (segment (start 117.54 87.46) (end 117.5 87.5) (width 0.2) (layer "F.Cu") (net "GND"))
 (segment (start 133 94.0875) (end 133 98) (width 0.2) (layer "F.Cu") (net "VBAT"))
 (segment (start 125.9125 87) (end 133 94.0875) (width 0.2) (layer "F.Cu") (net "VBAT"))
 (segment (start 133.476346 99.275) (end 132.323654 99.275) (width 0.2) (layer "F.Cu") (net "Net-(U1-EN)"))
 (segment (start 119.5 94) (end 120.6 92.9) (width 0.2) (layer "F.Cu") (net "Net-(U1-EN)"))
 (segment (start 131.65 98.601346) (end 131.65 97.398654) (width 0.2) (layer "F.Cu") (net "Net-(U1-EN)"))
 (segment (start 119.5 94.5) (end 119.45 94.55) (width 0.2) (layer "F.Cu") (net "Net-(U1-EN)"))
 (segment (start 131.65 97.398654) (end 130.751408 96.500062) (width 0.2) (layer "F.Cu") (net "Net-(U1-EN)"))
 (segment (start 141.05 84.25) (end 134.15 91.15) (width 0.2) (layer "F.Cu") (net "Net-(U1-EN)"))
 (segment (start 119.949938 96.500062) (end 119.45 97) (width 0.2) (layer "F.Cu") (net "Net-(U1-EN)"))
 (segment (start 120.04 85.03) (end 120.04 84.5) (width 0.2) (layer "F.Cu") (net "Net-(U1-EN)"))
 (segment (start 119.5 94) (end 119.5 94.5) (width 0.2) (layer "F.Cu") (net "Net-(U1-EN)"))
 (segment (start 134.15 98.601346) (end 133.476346 99.275) (width 0.2) (layer "F.Cu") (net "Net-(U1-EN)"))
 (segment (start 130.751408 96.500062) (end 119.949938 96.500062) (width 0.2) (layer "F.Cu") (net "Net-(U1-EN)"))
 (segment (start 134.15 91.15) (end 134.15 98.601346) (width 0.2) (layer "F.Cu") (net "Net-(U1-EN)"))
 (segment (start 119.45 94.55) (end 119.45 97) (width 0.2) (layer "F.Cu") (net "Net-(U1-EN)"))
 (segment (start 132.323654 99.275) (end 131.65 98.601346) (width 0.2) (layer "F.Cu") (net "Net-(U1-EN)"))
 (segment (start 156 66) (end 128.175 66) (width 0.2) (layer "F.Cu") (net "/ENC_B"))
 (segment (start 128.175 66) (end 126 63.825) (width 0.2) (layer "F.Cu") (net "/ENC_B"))
 (segment (start 141.05 74.05) (end 134.05 67.05) (width 0.2) (layer "F.Cu") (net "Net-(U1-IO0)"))
 (segment (start 141.05 75.75) (end 141.05 74.05) (width 0.2) (layer "F.Cu") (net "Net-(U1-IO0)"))
 (segment (start 128.1875 63.0125) (end 125.315256 63.0125) (width 0.2) (layer "F.Cu") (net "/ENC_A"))
 (segment (start 125 63.327756) (end 125 64.322244) (width 0.2) (layer "F.Cu") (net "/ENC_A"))
 (segment (start 125.315256 64.6375) (end 126.246814 64.6375) (width 0.2) (layer "F.Cu") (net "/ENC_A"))
 (segment (start 126.246814 64.6375) (end 127.7 66.090686) (width 0.2) (layer "F.Cu") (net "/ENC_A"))
 (segment (start 129 63.825) (end 128.1875 63.0125) (width 0.2) (layer "F.Cu") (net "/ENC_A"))
 (segment (start 140 63.5) (end 139.675 63.825) (width 0.2) (layer "F.Cu") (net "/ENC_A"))
 (segment (start 127.7 66.090686) (end 127.7 67.05) (width 0.2) (layer "F.Cu") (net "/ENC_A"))
 (segment (start 156 63.5) (end 140 63.5) (width 0.2) (layer "F.Cu") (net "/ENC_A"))
 (segment (start 125.315256 63.0125) (end 125 63.327756) (width 0.2) (layer "F.Cu") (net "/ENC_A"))
 (segment (start 139.675 63.825) (end 129 63.825) (width 0.2) (layer "F.Cu") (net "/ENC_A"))
 (segment (start 125 64.322244) (end 125.315256 64.6375) (width 0.2) (layer "F.Cu") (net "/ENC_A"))
 (segment (start 125.275 55.275) (end 124 54) (width 0.2) (layer "F.Cu") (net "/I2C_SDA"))
 (segment (start 138.5 54) (end 137.225 55.275) (width 0.2) (layer "F.Cu") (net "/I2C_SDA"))
 (segment (start 123.5 66.66) (end 123.89 67.05) (width 0.2) (layer "F.Cu") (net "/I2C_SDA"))
 (segment (start 137.225 55.275) (end 125.275 55.275) (width 0.2) (layer "F.Cu") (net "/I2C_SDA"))
 (segment (start 124 54) (end 124.5 54.5) (width 0.2) (layer "F.Cu") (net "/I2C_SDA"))
 (segment (start 124.5 54.5) (end 124.5 62.825) (width 0.2) (layer "F.Cu") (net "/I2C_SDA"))
 (segment (start 124.5 62.825) (end 123.5 63.825) (width 0.2) (layer "F.Cu") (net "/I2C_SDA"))
 (segment (start 123.5 63.825) (end 123.5 66.66) (width 0.2) (layer "F.Cu") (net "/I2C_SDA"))
 (segment (start 136 54) (end 134.725 52.725) (width 0.2) (layer "F.Cu") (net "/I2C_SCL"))
 (segment (start 121.5 54) (end 121.5 62.325) (width 0.2) (layer "F.Cu") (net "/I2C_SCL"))
 (segment (start 122.775 52.725) (end 121.5 54) (width 0.2) (layer "F.Cu") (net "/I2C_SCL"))
 (segment (start 121.5 62.325) (end 120 63.825) (width 0.2) (layer "F.Cu") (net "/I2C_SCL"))
 (segment (start 134.725 52.725) (end 122.775 52.725) (width 0.2) (layer "F.Cu") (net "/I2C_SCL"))
 (segment (start 120 66.97) (end 120.08 67.05) (width 0.2) (layer "F.Cu") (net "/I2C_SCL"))
 (segment (start 120 63.825) (end 120 66.97) (width 0.2) (layer "F.Cu") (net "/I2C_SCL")))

